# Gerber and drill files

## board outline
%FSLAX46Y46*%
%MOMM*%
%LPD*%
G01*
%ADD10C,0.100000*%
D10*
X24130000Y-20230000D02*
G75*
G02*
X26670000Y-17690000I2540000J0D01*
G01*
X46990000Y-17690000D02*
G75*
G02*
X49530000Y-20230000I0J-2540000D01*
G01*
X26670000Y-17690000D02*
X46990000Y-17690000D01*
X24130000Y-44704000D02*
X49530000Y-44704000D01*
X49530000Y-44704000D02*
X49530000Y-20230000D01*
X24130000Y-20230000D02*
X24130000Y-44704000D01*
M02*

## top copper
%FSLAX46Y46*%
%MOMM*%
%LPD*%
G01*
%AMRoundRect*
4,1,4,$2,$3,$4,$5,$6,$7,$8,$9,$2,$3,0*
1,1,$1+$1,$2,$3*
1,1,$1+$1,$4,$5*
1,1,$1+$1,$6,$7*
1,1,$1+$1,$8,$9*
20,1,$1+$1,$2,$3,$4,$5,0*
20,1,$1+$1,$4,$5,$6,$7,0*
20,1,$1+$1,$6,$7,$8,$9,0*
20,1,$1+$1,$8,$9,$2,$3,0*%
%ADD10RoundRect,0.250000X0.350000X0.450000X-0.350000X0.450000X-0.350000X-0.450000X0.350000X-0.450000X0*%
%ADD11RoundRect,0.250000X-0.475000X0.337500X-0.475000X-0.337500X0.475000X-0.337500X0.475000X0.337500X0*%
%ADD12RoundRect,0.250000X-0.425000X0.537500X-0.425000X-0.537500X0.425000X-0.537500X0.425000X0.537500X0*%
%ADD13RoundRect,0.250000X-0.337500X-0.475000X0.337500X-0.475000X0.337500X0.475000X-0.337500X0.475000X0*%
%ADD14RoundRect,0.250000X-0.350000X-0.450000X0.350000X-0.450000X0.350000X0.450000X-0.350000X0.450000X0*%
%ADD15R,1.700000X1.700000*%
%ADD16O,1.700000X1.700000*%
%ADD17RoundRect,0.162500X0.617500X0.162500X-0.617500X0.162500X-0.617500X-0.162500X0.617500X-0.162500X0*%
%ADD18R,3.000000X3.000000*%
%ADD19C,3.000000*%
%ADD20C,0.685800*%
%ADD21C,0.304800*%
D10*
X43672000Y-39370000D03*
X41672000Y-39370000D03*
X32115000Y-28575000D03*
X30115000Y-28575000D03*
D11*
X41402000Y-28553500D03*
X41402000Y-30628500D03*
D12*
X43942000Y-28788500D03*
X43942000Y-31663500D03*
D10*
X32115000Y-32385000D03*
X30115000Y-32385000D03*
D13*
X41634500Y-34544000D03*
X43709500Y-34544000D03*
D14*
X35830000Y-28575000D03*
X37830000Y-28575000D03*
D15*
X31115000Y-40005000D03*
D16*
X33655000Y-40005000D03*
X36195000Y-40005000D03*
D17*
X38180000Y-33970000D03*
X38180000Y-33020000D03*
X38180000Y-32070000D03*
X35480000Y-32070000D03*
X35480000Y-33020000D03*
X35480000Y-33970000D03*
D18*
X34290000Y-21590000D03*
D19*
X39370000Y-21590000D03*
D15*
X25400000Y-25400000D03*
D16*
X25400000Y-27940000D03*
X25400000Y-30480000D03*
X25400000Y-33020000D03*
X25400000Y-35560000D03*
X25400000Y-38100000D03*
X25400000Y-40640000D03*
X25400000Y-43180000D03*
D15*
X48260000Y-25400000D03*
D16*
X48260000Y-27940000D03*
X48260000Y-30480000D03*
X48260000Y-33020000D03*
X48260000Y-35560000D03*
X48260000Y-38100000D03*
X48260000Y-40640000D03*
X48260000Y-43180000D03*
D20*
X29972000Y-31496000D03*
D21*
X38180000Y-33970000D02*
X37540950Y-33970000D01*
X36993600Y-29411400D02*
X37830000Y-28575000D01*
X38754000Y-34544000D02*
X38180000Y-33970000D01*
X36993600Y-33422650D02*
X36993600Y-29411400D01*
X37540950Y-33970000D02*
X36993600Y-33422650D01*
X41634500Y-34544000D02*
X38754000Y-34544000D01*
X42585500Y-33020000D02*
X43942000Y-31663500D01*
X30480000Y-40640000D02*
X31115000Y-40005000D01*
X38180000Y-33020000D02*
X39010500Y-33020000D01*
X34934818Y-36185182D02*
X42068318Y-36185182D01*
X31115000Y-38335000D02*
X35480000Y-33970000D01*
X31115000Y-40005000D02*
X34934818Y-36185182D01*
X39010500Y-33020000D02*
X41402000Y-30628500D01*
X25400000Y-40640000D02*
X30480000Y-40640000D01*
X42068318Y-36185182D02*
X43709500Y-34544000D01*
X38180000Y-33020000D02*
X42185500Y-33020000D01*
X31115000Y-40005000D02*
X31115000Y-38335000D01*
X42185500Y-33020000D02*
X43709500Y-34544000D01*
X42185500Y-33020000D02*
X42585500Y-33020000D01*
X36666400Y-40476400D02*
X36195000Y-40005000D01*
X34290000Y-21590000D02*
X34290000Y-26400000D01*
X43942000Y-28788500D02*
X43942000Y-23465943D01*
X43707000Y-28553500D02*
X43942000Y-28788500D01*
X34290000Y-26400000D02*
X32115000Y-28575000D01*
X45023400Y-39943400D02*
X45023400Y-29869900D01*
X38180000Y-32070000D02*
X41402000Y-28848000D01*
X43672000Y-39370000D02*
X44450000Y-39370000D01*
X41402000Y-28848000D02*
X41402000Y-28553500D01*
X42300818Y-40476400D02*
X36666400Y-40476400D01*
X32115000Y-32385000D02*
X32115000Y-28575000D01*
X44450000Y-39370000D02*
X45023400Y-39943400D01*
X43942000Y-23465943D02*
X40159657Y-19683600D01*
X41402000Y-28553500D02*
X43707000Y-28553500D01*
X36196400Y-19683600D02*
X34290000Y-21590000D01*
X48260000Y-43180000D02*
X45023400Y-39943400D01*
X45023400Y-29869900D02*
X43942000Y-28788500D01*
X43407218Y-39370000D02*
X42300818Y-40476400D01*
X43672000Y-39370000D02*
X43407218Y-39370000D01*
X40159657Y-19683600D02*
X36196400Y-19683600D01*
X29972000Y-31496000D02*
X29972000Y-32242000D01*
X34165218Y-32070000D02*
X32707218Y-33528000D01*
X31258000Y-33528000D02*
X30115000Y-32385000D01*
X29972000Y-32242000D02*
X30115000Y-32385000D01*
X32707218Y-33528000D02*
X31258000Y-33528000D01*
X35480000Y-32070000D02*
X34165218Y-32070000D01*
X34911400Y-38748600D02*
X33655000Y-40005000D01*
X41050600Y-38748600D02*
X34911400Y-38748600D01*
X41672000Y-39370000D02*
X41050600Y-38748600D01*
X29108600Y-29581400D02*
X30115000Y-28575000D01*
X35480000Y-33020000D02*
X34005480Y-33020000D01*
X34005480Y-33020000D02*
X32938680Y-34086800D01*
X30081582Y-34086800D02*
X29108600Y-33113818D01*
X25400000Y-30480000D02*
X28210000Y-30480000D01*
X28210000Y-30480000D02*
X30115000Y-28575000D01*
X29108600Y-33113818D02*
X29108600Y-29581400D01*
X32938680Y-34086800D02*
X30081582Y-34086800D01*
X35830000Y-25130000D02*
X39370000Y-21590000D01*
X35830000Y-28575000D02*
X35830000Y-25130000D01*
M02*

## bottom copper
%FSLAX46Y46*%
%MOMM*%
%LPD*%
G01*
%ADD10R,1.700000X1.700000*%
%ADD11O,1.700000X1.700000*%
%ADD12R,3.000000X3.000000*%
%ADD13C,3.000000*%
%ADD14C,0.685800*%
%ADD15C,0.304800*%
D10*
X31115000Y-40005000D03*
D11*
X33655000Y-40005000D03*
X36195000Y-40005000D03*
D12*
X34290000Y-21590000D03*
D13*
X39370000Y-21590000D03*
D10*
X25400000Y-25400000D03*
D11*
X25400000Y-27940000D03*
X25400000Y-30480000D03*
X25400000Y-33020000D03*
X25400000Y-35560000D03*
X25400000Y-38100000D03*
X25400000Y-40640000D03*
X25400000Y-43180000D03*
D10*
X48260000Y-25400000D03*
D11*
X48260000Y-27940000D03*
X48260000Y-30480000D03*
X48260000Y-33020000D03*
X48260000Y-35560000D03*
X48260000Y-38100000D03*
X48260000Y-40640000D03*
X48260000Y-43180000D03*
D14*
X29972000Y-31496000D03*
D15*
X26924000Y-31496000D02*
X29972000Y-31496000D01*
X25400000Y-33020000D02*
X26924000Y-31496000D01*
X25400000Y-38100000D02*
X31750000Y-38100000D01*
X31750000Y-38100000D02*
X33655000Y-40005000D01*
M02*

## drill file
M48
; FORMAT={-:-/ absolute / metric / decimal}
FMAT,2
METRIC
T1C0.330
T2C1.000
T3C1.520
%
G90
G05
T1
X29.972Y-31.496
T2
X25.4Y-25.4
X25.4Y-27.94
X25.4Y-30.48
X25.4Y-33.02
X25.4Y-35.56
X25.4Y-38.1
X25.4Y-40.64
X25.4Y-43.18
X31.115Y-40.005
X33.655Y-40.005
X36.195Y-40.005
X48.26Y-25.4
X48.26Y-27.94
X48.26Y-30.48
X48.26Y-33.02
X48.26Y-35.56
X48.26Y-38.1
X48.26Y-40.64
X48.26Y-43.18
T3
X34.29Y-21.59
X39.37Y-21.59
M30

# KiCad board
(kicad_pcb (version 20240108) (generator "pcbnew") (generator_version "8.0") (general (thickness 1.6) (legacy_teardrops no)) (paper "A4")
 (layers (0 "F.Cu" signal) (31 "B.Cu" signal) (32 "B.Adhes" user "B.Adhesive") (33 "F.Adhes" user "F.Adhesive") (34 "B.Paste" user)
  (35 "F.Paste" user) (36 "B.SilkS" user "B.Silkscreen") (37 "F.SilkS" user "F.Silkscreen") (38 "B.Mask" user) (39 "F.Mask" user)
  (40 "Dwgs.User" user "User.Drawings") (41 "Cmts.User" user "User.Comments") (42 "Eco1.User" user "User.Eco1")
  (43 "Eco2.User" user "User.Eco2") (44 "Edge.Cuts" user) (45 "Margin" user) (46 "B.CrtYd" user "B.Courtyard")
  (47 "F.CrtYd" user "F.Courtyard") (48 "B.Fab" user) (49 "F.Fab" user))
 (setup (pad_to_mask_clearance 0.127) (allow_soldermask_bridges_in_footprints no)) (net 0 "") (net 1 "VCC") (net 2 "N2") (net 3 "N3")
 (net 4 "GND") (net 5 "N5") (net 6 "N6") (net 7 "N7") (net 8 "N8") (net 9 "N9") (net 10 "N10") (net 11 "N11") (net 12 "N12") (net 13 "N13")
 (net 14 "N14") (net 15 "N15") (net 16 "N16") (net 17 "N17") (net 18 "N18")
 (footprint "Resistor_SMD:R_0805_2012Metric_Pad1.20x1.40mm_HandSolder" (layer "F.Cu") (at 42.672 39.37 180)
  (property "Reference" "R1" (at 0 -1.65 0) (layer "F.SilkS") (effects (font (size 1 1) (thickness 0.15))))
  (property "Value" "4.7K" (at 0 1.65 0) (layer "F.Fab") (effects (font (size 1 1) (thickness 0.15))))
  (pad "1" smd roundrect (at -1 0 180) (size 1.2 1.4) (layers "F.Cu" "F.Paste" "F.Mask") (roundrect_rratio 0.208333) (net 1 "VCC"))
  (pad "2" smd roundrect (at 1 0 180) (size 1.2 1.4) (layers "F.Cu" "F.Paste" "F.Mask") (roundrect_rratio 0.208333) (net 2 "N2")))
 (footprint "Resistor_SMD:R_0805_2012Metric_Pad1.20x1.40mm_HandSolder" (layer "F.Cu") (at 31.115 28.575 180)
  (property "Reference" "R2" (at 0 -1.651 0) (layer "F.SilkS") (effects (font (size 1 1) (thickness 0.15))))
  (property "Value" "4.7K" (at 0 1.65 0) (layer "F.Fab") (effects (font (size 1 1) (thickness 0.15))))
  (pad "1" smd roundrect (at -1 0 180) (size 1.2 1.4) (layers "F.Cu" "F.Paste" "F.Mask") (roundrect_rratio 0.208333) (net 1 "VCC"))
  (pad "2" smd roundrect (at 1 0 180) (size 1.2 1.4) (layers "F.Cu" "F.Paste" "F.Mask") (roundrect_rratio 0.208333) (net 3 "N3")))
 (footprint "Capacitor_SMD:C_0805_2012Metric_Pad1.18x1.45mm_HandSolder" (layer "F.Cu") (at 41.402 29.591 -90)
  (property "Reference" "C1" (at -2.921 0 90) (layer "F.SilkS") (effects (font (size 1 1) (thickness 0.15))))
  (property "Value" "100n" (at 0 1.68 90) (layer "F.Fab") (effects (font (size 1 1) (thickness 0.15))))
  (pad "1" smd roundrect (at -1.0375 0 270) (size 1.175 1.45) (layers "F.Cu" "F.Paste" "F.Mask") (roundrect_rratio 0.212766) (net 1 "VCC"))
  (pad "2" smd roundrect (at 1.0375 0 270) (size 1.175 1.45) (layers "F.Cu" "F.Paste" "F.Mask") (roundrect_rratio 0.212766) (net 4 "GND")))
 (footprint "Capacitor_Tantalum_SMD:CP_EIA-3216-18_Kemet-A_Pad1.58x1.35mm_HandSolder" (layer "F.Cu") (at 43.942 30.226 -90)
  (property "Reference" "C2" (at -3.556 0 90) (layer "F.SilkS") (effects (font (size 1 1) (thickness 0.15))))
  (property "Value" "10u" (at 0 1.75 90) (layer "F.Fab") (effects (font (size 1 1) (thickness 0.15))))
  (pad "1" smd roundrect (at -1.4375 0 270) (size 1.575 1.35) (layers "F.Cu" "F.Paste" "F.Mask") (roundrect_rratio 0.185185) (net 1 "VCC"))
  (pad "2" smd roundrect (at 1.4375 0 270) (size 1.575 1.35) (layers "F.Cu" "F.Paste" "F.Mask") (roundrect_rratio 0.185185) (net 4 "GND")))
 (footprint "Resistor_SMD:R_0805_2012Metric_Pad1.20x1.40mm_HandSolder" (layer "F.Cu") (at 31.115 32.385 180)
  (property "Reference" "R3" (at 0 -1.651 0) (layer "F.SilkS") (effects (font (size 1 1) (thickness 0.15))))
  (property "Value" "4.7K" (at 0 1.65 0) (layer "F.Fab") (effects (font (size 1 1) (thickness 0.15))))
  (pad "1" smd roundrect (at -1 0 180) (size 1.2 1.4) (layers "F.Cu" "F.Paste" "F.Mask") (roundrect_rratio 0.208333) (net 1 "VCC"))
  (pad "2" smd roundrect (at 1 0 180) (size 1.2 1.4) (layers "F.Cu" "F.Paste" "F.Mask") (roundrect_rratio 0.208333) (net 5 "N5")))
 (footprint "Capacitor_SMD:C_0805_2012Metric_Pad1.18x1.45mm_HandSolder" (layer "F.Cu") (at 42.672 34.544)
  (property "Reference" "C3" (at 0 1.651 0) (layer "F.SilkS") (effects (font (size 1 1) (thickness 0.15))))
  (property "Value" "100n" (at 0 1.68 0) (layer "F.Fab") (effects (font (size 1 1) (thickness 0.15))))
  (pad "1" smd roundrect (at -1.0375 0) (size 1.175 1.45) (layers "F.Cu" "F.Paste" "F.Mask") (roundrect_rratio 0.212766) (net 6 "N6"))
  (pad "2" smd roundrect (at 1.0375 0) (size 1.175 1.45) (layers "F.Cu" "F.Paste" "F.Mask") (roundrect_rratio 0.212766) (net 4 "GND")))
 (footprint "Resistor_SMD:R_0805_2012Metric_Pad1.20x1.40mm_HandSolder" (layer "F.Cu") (at 36.83 28.575)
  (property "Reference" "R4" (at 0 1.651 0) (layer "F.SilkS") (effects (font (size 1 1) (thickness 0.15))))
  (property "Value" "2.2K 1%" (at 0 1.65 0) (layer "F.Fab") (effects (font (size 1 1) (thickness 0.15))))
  (pad "1" smd roundrect (at -1 0) (size 1.2 1.4) (layers "F.Cu" "F.Paste" "F.Mask") (roundrect_rratio 0.208333) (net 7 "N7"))
  (pad "2" smd roundrect (at 1 0) (size 1.2 1.4) (layers "F.Cu" "F.Paste" "F.Mask") (roundrect_rratio 0.208333) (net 6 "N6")))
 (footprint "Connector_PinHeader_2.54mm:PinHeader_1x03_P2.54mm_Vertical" (layer "F.Cu") (at 31.115 40.005 90)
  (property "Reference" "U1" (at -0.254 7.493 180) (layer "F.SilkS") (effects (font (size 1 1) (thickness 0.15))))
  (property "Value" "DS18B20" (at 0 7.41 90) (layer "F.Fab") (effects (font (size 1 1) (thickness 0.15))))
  (pad "1" thru_hole rect (at 0 0 90) (size 1.7 1.7) (drill 1) (layers "*.Cu" "*.Mask") (remove_unused_layers no) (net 4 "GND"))
  (pad "2" thru_hole oval (at 0 2.54 90) (size 1.7 1.7) (drill 1) (layers "*.Cu" "*.Mask") (remove_unused_layers no) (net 2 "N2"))
  (pad "3" thru_hole oval (at 0 5.08 90) (size 1.7 1.7) (drill 1) (layers "*.Cu" "*.Mask") (remove_unused_layers no) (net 1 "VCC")))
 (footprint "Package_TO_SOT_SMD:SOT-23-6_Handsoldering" (layer "F.Cu") (at 36.83 33.02 180)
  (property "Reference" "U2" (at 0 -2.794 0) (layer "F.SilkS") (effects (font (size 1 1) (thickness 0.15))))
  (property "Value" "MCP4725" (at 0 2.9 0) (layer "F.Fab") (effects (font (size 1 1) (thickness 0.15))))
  (pad "1" smd roundrect (at -1.35 -0.95 180) (size 1.56 0.65) (layers "F.Cu" "F.Paste" "F.Mask") (roundrect_rratio 0.25) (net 6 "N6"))
  (pad "2" smd roundrect (at -1.35 0 180) (size 1.56 0.65) (layers "F.Cu" "F.Paste" "F.Mask") (roundrect_rratio 0.25) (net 4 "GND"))
  (pad "3" smd roundrect (at -1.35 0.95 180) (size 1.56 0.65) (layers "F.Cu" "F.Paste" "F.Mask") (roundrect_rratio 0.25) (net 1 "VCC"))
  (pad "4" smd roundrect (at 1.35 0.95 180) (size 1.56 0.65) (layers "F.Cu" "F.Paste" "F.Mask") (roundrect_rratio 0.25) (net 5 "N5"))
  (pad "5" smd roundrect (at 1.35 0 180) (size 1.56 0.65) (layers "F.Cu" "F.Paste" "F.Mask") (roundrect_rratio 0.25) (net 3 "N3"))
  (pad "6" smd roundrect (at 1.35 -0.95 180) (size 1.56 0.65) (layers "F.Cu" "F.Paste" "F.Mask") (roundrect_rratio 0.25) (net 4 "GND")))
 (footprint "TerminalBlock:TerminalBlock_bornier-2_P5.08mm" (layer "F.Cu") (at 34.29 21.59)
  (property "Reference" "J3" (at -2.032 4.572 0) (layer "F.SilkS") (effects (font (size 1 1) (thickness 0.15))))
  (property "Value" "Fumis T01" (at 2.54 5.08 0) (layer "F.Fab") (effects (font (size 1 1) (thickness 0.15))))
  (pad "1" thru_hole rect (at 0 0) (size 3 3) (drill 1.52) (layers "*.Cu" "*.Mask") (remove_unused_layers no) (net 1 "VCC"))
  (pad "2" thru_hole circle (at 5.08 0) (size 3 3) (drill 1.52) (layers "*.Cu" "*.Mask") (remove_unused_layers no) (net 7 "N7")))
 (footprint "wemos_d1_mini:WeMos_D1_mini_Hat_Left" (layer "B.Cu") (at 25.4 25.4 180)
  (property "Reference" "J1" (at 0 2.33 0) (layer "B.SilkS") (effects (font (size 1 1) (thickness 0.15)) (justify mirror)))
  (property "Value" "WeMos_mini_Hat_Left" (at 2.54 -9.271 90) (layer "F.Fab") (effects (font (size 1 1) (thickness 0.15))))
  (pad "1" thru_hole rect (at 0 0 180) (size 1.7 1.7) (drill 1) (layers "*.Cu" "*.Mask") (remove_unused_layers no) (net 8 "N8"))
  (pad "2" thru_hole oval (at 0 -2.54 180) (size 1.7 1.7) (drill 1) (layers "*.Cu" "*.Mask") (remove_unused_layers no) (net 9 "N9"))
  (pad "3" thru_hole oval (at 0 -5.08 180) (size 1.7 1.7) (drill 1) (layers "*.Cu" "*.Mask") (remove_unused_layers no) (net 3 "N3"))
  (pad "4" thru_hole oval (at 0 -7.62 180) (size 1.7 1.7) (drill 1) (layers "*.Cu" "*.Mask") (remove_unused_layers no) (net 5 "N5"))
  (pad "5" thru_hole oval (at 0 -10.16 180) (size 1.7 1.7) (drill 1) (layers "*.Cu" "*.Mask") (remove_unused_layers no) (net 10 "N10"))
  (pad "6" thru_hole oval (at 0 -12.7 180) (size 1.7 1.7) (drill 1) (layers "*.Cu" "*.Mask") (remove_unused_layers no) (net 2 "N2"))
  (pad "7" thru_hole oval (at 0 -15.24 180) (size 1.7 1.7) (drill 1) (layers "*.Cu" "*.Mask") (remove_unused_layers no) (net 4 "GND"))
  (pad "8" thru_hole oval (at 0 -17.78 180) (size 1.7 1.7) (drill 1) (layers "*.Cu" "*.Mask") (remove_unused_layers no) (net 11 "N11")))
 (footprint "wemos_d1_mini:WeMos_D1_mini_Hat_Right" (layer "B.Cu") (at 48.26 25.4 180)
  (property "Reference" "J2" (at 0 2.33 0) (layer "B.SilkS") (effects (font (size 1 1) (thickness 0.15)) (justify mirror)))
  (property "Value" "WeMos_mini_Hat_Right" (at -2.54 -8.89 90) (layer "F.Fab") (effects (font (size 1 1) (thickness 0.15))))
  (pad "1" thru_hole rect (at 0 0 180) (size 1.7 1.7) (drill 1) (layers "*.Cu" "*.Mask") (remove_unused_layers no) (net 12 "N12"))
  (pad "2" thru_hole oval (at 0 -2.54 180) (size 1.7 1.7) (drill 1) (layers "*.Cu" "*.Mask") (remove_unused_layers no) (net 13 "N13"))
  (pad "3" thru_hole oval (at 0 -5.08 180) (size 1.7 1.7) (drill 1) (layers "*.Cu" "*.Mask") (remove_unused_layers no) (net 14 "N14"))
  (pad "4" thru_hole oval (at 0 -7.62 180) (size 1.7 1.7) (drill 1) (layers "*.Cu" "*.Mask") (remove_unused_layers no) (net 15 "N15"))
  (pad "5" thru_hole oval (at 0 -10.16 180) (size 1.7 1.7) (drill 1) (layers "*.Cu" "*.Mask") (remove_unused_layers no) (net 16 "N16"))
  (pad "6" thru_hole oval (at 0 -12.7 180) (size 1.7 1.7) (drill 1) (layers "*.Cu" "*.Mask") (remove_unused_layers no) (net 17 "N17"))
  (pad "7" thru_hole oval (at 0 -15.24 180) (size 1.7 1.7) (drill 1) (layers "*.Cu" "*.Mask") (remove_unused_layers no) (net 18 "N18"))
  (pad "8" thru_hole oval (at 0 -17.78 180) (size 1.7 1.7) (drill 1) (layers "*.Cu" "*.Mask") (remove_unused_layers no) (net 1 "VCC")))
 (gr_arc (start 24.13 20.23) (mid 24.873949 18.433949) (end 26.67 17.69) (stroke (width 0.1) (type default)) (layer "Edge.Cuts"))
 (gr_arc (start 46.99 17.69) (mid 48.786051 18.433949) (end 49.53 20.23) (stroke (width 0.1) (type default)) (layer "Edge.Cuts"))
 (gr_line (start 26.67 17.69) (end 46.99 17.69) (stroke (width 0.1) (type default)) (layer "Edge.Cuts"))
 (gr_line (start 24.13 44.704) (end 49.53 44.704) (stroke (width 0.1) (type default)) (layer "Edge.Cuts"))
 (gr_line (start 49.53 44.704) (end 49.53 20.23) (stroke (width 0.1) (type default)) (layer "Edge.Cuts"))
 (gr_line (start 24.13 20.23) (end 24.13 44.704) (stroke (width 0.1) (type default)) (layer "Edge.Cuts"))
 (segment (start 38.18 33.97) (end 37.54095 33.97) (width 0.3048) (layer "F.Cu") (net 6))
 (segment (start 36.9936 29.4114) (end 37.83 28.575) (width 0.3048) (layer "F.Cu") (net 6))
 (segment (start 38.754 34.544) (end 38.18 33.97) (width 0.3048) (layer "F.Cu") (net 6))
 (segment (start 36.9936 33.42265) (end 36.9936 29.4114) (width 0.3048) (layer "F.Cu") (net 6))
 (segment (start 37.54095 33.97) (end 36.9936 33.42265) (width 0.3048) (layer "F.Cu") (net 6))
 (segment (start 41.6345 34.544) (end 38.754 34.544) (width 0.3048) (layer "F.Cu") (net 6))
 (segment (start 42.5855 33.02) (end 43.942 31.6635) (width 0.3048) (layer "F.Cu") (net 4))
 (segment (start 30.48 40.64) (end 31.115 40.005) (width 0.3048) (layer "F.Cu") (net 4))
 (segment (start 38.18 33.02) (end 39.0105 33.02) (width 0.3048) (layer "F.Cu") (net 4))
 (segment (start 34.934818 36.185182) (end 42.068318 36.185182) (width 0.3048) (layer "F.Cu") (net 4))
 (segment (start 31.115 38.335) (end 35.48 33.97) (width 0.3048) (layer "F.Cu") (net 4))
 (segment (start 31.115 40.005) (end 34.934818 36.185182) (width 0.3048) (layer "F.Cu") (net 4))
 (segment (start 39.0105 33.02) (end 41.402 30.6285) (width 0.3048) (layer "F.Cu") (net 4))
 (segment (start 25.4 40.64) (end 30.48 40.64) (width 0.3048) (layer "F.Cu") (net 4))
 (segment (start 42.068318 36.185182) (end 43.7095 34.544) (width 0.3048) (layer "F.Cu") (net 4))
 (segment (start 38.18 33.02) (end 42.1855 33.02) (width 0.3048) (layer "F.Cu") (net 4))
 (segment (start 31.115 40.005) (end 31.115 38.335) (width 0.3048) (layer "F.Cu") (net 4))
 (segment (start 42.1855 33.02) (end 43.7095 34.544) (width 0.3048) (layer "F.Cu") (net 4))
 (segment (start 42.1855 33.02) (end 42.5855 33.02) (width 0.3048) (layer "F.Cu") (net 4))
 (segment (start 36.6664 40.4764) (end 36.195 40.005) (width 0.3048) (layer "F.Cu") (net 1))
 (segment (start 34.29 21.59) (end 34.29 26.4) (width 0.3048) (layer "F.Cu") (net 1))
 (segment (start 43.942 28.7885) (end 43.942 23.465943) (width 0.3048) (layer "F.Cu") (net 1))
 (segment (start 43.707 28.5535) (end 43.942 28.7885) (width 0.3048) (layer "F.Cu") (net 1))
 (segment (start 34.29 26.4) (end 32.115 28.575) (width 0.3048) (layer "F.Cu") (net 1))
 (segment (start 45.0234 39.9434) (end 45.0234 29.8699) (width 0.3048) (layer "F.Cu") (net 1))
 (segment (start 38.18 32.07) (end 41.402 28.848) (width 0.3048) (layer "F.Cu") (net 1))
 (segment (start 43.672 39.37) (end 44.45 39.37) (width 0.3048) (layer "F.Cu") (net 1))
 (segment (start 41.402 28.848) (end 41.402 28.5535) (width 0.3048) (layer "F.Cu") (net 1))
 (segment (start 42.300818 40.4764) (end 36.6664 40.4764) (width 0.3048) (layer "F.Cu") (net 1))
 (segment (start 32.115 32.385) (end 32.115 28.575) (width 0.3048) (layer "F.Cu") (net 1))
 (segment (start 44.45 39.37) (end 45.0234 39.9434) (width 0.3048) (layer "F.Cu") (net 1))
 (segment (start 43.942 23.465943) (end 40.159657 19.6836) (width 0.3048) (layer "F.Cu") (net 1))
 (segment (start 41.402 28.5535) (end 43.707 28.5535) (width 0.3048) (layer "F.Cu") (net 1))
 (segment (start 36.1964 19.6836) (end 34.29 21.59) (width 0.3048) (layer "F.Cu") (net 1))
 (segment (start 48.26 43.18) (end 45.0234 39.9434) (width 0.3048) (layer "F.Cu") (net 1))
 (segment (start 45.0234 29.8699) (end 43.942 28.7885) (width 0.3048) (layer "F.Cu") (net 1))
 (segment (start 43.407218 39.37) (end 42.300818 40.4764) (width 0.3048) (layer "F.Cu") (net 1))
 (segment (start 43.672 39.37) (end 43.407218 39.37) (width 0.3048) (layer "F.Cu") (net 1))
 (segment (start 40.159657 19.6836) (end 36.1964 19.6836) (width 0.3048) (layer "F.Cu") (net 1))
 (segment (start 29.972 31.496) (end 29.972 32.242) (width 0.3048) (layer "F.Cu") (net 5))
 (segment (start 34.165218 32.07) (end 32.707218 33.528) (width 0.3048) (layer "F.Cu") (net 5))
 (segment (start 31.258 33.528) (end 30.115 32.385) (width 0.3048) (layer "F.Cu") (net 5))
 (segment (start 29.972 32.242) (end 30.115 32.385) (width 0.3048) (layer "F.Cu") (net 5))
 (segment (start 32.707218 33.528) (end 31.258 33.528) (width 0.3048) (layer "F.Cu") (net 5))
 (segment (start 35.48 32.07) (end 34.165218 32.07) (width 0.3048) (layer "F.Cu") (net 5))
 (via (at 29.972 31.496) (size 0.6858) (drill 0.3302) (layers "F.Cu" "B.Cu") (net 5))
 (segment (start 26.924 31.496) (end 29.972 31.496) (width 0.3048) (layer "B.Cu") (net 5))
 (segment (start 25.4 33.02) (end 26.924 31.496) (width 0.3048) (layer "B.Cu") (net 5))
 (segment (start 34.9114 38.7486) (end 33.655 40.005) (width 0.3048) (layer "F.Cu") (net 2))
 (segment (start 41.0506 38.7486) (end 34.9114 38.7486) (width 0.3048) (layer "F.Cu") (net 2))
 (segment (start 41.672 39.37) (end 41.0506 38.7486) (width 0.3048) (layer "F.Cu") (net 2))
 (segment (start 25.4 38.1) (end 31.75 38.1) (width 0.3048) (layer "B.Cu") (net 2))
 (segment (start 31.75 38.1) (end 33.655 40.005) (width 0.3048) (layer "B.Cu") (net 2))
 (segment (start 29.1086 29.5814) (end 30.115 28.575) (width 0.3048) (layer "F.Cu") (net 3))
 (segment (start 35.48 33.02) (end 34.00548 33.02) (width 0.3048) (layer "F.Cu") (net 3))
 (segment (start 34.00548 33.02) (end 32.93868 34.0868) (width 0.3048) (layer "F.Cu") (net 3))
 (segment (start 30.081582 34.0868) (end 29.1086 33.113818) (width 0.3048) (layer "F.Cu") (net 3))
 (segment (start 25.4 30.48) (end 28.21 30.48) (width 0.3048) (layer "F.Cu") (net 3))
 (segment (start 28.21 30.48) (end 30.115 28.575) (width 0.3048) (layer "F.Cu") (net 3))
 (segment (start 29.1086 33.113818) (end 29.1086 29.5814) (width 0.3048) (layer "F.Cu") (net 3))
 (segment (start 32.93868 34.0868) (end 30.081582 34.0868) (width 0.3048) (layer "F.Cu") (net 3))
 (segment (start 35.83 25.13) (end 39.37 21.59) (width 0.3048) (layer "F.Cu") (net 7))
 (segment (start 35.83 28.575) (end 35.83 25.13) (width 0.3048) (layer "F.Cu") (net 7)))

